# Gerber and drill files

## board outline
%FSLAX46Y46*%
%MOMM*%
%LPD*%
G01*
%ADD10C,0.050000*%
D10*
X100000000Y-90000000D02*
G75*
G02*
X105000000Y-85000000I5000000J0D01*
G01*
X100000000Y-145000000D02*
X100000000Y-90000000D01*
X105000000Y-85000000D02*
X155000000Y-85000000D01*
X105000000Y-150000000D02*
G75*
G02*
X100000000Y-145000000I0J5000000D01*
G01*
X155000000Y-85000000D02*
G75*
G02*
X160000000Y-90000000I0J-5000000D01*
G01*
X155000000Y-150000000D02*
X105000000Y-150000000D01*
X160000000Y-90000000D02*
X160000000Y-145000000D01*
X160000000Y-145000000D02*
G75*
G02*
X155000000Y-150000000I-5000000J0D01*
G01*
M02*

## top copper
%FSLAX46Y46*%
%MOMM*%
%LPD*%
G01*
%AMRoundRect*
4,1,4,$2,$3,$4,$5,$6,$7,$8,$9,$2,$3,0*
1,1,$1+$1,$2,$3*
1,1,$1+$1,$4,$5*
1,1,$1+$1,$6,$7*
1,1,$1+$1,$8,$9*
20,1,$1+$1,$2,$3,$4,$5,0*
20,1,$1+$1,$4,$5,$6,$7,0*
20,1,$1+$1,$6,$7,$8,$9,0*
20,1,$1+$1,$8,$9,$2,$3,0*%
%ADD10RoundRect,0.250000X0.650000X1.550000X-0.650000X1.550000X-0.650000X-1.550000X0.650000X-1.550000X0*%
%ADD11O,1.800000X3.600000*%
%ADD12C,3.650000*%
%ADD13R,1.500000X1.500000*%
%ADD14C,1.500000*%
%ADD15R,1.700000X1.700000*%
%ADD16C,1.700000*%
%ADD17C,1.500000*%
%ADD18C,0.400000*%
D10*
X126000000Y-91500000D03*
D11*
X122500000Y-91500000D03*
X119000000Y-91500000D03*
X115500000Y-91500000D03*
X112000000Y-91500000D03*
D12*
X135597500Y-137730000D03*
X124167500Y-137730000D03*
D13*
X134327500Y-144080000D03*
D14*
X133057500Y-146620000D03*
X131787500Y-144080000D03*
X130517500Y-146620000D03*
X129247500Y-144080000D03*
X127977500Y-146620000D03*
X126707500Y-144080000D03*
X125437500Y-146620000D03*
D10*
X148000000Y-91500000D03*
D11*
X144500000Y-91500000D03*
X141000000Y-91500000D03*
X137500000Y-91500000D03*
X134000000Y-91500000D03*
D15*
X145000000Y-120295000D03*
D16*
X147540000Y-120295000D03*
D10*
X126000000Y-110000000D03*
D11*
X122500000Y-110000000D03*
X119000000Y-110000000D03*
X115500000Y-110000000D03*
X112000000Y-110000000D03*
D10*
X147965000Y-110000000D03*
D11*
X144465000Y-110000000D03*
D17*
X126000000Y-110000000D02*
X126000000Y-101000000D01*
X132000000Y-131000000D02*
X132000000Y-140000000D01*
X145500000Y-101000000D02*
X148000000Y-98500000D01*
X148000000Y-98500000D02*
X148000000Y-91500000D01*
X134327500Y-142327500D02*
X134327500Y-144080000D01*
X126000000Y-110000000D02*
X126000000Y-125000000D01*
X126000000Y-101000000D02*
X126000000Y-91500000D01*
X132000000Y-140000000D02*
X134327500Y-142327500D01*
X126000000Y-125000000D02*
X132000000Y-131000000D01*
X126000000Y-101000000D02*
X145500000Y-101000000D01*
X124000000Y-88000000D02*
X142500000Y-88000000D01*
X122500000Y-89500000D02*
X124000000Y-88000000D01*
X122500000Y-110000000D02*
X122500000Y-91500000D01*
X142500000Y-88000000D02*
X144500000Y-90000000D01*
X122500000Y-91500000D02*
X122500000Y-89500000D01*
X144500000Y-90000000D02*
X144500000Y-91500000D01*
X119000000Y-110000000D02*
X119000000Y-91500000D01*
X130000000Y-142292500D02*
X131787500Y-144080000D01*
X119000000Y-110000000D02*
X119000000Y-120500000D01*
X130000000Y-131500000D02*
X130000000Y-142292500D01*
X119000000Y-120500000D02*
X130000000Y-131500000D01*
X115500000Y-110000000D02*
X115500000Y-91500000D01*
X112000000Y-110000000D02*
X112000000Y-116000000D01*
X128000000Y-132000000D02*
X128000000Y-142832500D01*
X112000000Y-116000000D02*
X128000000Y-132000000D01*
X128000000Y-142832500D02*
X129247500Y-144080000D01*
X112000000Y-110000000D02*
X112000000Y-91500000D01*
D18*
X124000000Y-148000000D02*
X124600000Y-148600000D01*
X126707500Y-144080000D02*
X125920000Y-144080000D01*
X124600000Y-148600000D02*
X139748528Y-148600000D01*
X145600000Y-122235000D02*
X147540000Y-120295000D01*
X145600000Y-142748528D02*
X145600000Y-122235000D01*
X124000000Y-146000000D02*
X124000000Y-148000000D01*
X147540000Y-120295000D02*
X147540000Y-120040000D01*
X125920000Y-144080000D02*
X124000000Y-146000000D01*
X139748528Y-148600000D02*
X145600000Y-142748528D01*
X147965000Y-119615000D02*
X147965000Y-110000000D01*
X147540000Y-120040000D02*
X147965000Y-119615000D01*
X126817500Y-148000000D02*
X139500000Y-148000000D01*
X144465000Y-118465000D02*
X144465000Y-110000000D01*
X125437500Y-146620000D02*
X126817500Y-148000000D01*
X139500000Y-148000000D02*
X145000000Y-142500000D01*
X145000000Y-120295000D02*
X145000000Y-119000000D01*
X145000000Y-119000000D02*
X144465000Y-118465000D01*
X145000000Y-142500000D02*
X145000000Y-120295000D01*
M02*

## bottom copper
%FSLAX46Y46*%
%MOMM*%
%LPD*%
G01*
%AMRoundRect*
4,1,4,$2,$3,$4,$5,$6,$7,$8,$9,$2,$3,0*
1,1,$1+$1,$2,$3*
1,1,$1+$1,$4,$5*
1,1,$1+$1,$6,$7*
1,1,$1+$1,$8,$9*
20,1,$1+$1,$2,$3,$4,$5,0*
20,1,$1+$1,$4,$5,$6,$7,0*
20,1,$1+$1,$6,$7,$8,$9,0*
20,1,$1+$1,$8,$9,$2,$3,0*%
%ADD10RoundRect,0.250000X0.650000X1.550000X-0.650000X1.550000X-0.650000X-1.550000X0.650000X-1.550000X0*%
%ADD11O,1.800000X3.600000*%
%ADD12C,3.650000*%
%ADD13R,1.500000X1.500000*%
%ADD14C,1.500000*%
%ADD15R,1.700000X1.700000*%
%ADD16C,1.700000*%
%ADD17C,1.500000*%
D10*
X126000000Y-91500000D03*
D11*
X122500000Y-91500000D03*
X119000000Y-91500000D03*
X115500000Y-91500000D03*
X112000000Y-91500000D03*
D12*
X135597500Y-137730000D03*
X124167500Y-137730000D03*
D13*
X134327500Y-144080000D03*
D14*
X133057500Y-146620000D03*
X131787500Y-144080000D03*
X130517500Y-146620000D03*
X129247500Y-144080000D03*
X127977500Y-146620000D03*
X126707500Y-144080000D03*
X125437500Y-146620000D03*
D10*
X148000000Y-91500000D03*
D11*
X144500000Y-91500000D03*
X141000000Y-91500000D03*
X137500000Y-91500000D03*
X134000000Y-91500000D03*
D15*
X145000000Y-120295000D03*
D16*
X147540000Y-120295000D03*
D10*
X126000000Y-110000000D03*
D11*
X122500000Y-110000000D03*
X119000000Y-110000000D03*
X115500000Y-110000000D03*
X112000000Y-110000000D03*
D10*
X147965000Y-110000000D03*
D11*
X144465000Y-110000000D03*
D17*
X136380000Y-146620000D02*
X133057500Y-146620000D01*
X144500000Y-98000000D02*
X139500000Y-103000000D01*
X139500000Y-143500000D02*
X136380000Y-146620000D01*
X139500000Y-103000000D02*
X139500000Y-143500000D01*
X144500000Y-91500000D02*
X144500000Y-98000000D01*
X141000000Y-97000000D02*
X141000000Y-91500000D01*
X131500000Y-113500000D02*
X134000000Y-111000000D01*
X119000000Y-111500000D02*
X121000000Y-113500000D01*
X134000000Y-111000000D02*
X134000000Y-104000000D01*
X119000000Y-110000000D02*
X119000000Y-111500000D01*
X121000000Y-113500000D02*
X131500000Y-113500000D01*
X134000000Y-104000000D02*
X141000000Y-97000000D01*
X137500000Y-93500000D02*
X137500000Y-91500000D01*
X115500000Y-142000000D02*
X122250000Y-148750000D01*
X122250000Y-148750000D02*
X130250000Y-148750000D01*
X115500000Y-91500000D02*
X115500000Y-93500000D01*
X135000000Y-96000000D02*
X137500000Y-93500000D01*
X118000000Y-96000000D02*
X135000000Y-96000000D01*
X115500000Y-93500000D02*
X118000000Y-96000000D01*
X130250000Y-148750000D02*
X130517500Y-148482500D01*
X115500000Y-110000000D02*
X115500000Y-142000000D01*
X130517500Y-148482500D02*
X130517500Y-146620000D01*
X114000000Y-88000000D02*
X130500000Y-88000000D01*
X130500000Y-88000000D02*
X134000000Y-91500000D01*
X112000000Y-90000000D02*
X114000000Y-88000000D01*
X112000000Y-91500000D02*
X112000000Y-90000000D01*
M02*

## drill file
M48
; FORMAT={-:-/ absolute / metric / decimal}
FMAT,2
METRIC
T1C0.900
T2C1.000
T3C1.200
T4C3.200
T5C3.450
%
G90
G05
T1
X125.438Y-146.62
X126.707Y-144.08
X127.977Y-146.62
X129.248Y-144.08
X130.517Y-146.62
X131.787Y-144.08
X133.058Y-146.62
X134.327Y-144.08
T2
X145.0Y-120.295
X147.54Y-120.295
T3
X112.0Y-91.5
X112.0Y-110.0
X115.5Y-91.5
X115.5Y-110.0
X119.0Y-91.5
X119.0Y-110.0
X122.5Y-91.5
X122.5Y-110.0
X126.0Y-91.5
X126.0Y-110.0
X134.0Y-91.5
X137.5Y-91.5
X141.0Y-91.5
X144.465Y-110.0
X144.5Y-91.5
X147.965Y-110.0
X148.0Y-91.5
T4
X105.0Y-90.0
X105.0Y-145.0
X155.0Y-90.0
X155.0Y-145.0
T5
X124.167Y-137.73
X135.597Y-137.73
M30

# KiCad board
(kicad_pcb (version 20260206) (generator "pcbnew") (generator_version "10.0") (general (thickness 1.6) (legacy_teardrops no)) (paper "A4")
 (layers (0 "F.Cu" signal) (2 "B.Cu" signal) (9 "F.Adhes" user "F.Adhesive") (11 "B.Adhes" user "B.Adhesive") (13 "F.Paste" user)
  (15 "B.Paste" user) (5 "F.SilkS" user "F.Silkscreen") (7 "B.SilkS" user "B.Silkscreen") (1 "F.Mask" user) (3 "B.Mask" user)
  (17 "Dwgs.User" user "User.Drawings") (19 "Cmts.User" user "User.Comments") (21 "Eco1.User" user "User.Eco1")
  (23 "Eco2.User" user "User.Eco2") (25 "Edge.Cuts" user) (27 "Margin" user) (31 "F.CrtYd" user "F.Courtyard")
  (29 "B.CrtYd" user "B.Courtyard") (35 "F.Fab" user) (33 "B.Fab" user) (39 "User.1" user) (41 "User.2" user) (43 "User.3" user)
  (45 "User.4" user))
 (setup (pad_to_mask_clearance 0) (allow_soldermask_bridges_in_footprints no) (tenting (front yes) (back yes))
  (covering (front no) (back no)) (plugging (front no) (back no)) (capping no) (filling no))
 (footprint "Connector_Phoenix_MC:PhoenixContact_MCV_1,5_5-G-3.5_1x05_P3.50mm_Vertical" (layer "F.Cu") (at 126 91.5 180)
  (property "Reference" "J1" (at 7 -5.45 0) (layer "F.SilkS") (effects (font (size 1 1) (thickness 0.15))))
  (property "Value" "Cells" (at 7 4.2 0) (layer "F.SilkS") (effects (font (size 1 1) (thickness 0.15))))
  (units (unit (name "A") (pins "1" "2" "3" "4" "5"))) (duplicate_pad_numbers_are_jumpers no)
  (pad "1" thru_hole roundrect (at 0 0 180) (size 1.8 3.6) (drill 1.2) (layers "*.Cu" "*.Mask") (remove_unused_layers no)
   (roundrect_rratio 0.138889) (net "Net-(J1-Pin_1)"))
  (pad "2" thru_hole oval (at 3.5 0 180) (size 1.8 3.6) (drill 1.2) (layers "*.Cu" "*.Mask") (remove_unused_layers no)
   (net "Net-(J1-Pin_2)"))
  (pad "3" thru_hole oval (at 7 0 180) (size 1.8 3.6) (drill 1.2) (layers "*.Cu" "*.Mask") (remove_unused_layers no) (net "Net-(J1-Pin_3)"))
  (pad "4" thru_hole oval (at 10.5 0 180) (size 1.8 3.6) (drill 1.2) (layers "*.Cu" "*.Mask") (remove_unused_layers no)
   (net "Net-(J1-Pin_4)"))
  (pad "5" thru_hole oval (at 14 0 180) (size 1.8 3.6) (drill 1.2) (layers "*.Cu" "*.Mask") (remove_unused_layers no) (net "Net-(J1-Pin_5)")))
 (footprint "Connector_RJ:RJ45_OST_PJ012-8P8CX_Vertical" (layer "F.Cu") (at 134.3275 144.08 180)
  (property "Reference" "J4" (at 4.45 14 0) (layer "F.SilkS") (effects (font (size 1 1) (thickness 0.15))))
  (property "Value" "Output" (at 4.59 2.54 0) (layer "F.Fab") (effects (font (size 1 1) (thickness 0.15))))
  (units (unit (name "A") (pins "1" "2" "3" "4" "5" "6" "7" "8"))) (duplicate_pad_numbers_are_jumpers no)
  (pad "" np_thru_hole circle (at -1.27 6.35 180) (size 3.65 3.65) (drill 3.45) (layers "*.Cu" "*.SilkS" "*.Mask"))
  (pad "" np_thru_hole circle (at 10.16 6.35 180) (size 3.65 3.65) (drill 3.45) (layers "*.Cu" "*.SilkS" "*.Mask"))
  (pad "1" thru_hole rect (at 0 0 180) (size 1.5 1.5) (drill 0.9) (layers "*.Cu" "*.Mask") (remove_unused_layers no) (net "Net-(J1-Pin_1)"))
  (pad "2" thru_hole circle (at 1.27 -2.54 180) (size 1.5 1.5) (drill 0.9) (layers "*.Cu" "*.Mask") (remove_unused_layers no)
   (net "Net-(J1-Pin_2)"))
  (pad "3" thru_hole circle (at 2.54 0 180) (size 1.5 1.5) (drill 0.9) (layers "*.Cu" "*.Mask") (remove_unused_layers no)
   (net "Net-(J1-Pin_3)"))
  (pad "4" thru_hole circle (at 3.81 -2.54 180) (size 1.5 1.5) (drill 0.9) (layers "*.Cu" "*.Mask") (remove_unused_layers no)
   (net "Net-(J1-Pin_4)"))
  (pad "5" thru_hole circle (at 5.08 0 180) (size 1.5 1.5) (drill 0.9) (layers "*.Cu" "*.Mask") (remove_unused_layers no)
   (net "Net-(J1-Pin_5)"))
  (pad "6" thru_hole circle (at 6.35 -2.54 180) (size 1.5 1.5) (drill 0.9) (layers "*.Cu" "*.Mask") (remove_unused_layers no)
   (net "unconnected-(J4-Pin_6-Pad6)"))
  (pad "7" thru_hole circle (at 7.62 0 180) (size 1.5 1.5) (drill 0.9) (layers "*.Cu" "*.Mask") (remove_unused_layers no)
   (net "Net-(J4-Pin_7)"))
  (pad "8" thru_hole circle (at 8.89 -2.54 180) (size 1.5 1.5) (drill 0.9) (layers "*.Cu" "*.Mask") (remove_unused_layers no)
   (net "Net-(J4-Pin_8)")))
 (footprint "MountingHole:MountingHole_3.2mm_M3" (layer "F.Cu") (at 105 145)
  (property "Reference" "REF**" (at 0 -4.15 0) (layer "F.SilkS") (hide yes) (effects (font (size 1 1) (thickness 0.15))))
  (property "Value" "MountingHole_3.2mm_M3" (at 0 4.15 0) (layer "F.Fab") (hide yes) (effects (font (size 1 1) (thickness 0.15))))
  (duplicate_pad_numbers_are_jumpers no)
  (pad "" np_thru_hole circle (at 0 0) (size 3.2 3.2) (drill 3.2) (layers "*.Cu" "*.Mask")))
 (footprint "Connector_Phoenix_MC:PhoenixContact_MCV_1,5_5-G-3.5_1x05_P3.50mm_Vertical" (layer "F.Cu") (at 148 91.5 180)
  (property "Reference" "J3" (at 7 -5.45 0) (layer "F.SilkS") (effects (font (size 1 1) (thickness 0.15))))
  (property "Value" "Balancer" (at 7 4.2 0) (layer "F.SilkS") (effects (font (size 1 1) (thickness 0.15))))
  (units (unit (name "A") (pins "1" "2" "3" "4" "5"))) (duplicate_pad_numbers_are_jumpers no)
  (pad "1" thru_hole roundrect (at 0 0 180) (size 1.8 3.6) (drill 1.2) (layers "*.Cu" "*.Mask") (remove_unused_layers no)
   (roundrect_rratio 0.138889) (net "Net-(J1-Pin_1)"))
  (pad "2" thru_hole oval (at 3.5 0 180) (size 1.8 3.6) (drill 1.2) (layers "*.Cu" "*.Mask") (remove_unused_layers no)
   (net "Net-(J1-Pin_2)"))
  (pad "3" thru_hole oval (at 7 0 180) (size 1.8 3.6) (drill 1.2) (layers "*.Cu" "*.Mask") (remove_unused_layers no) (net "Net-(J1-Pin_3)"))
  (pad "4" thru_hole oval (at 10.5 0 180) (size 1.8 3.6) (drill 1.2) (layers "*.Cu" "*.Mask") (remove_unused_layers no)
   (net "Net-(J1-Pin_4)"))
  (pad "5" thru_hole oval (at 14 0 180) (size 1.8 3.6) (drill 1.2) (layers "*.Cu" "*.Mask") (remove_unused_layers no) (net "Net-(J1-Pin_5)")))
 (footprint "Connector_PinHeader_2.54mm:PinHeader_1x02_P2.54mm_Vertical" (layer "F.Cu") (at 145 120.295 90)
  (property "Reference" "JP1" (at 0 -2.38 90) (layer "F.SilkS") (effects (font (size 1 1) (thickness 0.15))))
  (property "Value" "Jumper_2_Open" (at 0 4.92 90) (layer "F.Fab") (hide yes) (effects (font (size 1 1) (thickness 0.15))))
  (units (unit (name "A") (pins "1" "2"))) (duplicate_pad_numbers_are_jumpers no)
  (pad "1" thru_hole rect (at 0 0 90) (size 1.7 1.7) (drill 1) (layers "*.Cu" "*.Mask") (remove_unused_layers no) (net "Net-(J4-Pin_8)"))
  (pad "2" thru_hole circle (at 0 2.54 90) (size 1.7 1.7) (drill 1) (layers "*.Cu" "*.Mask") (remove_unused_layers no)
   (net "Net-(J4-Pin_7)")))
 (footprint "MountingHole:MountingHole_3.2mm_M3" (layer "F.Cu") (at 105 90)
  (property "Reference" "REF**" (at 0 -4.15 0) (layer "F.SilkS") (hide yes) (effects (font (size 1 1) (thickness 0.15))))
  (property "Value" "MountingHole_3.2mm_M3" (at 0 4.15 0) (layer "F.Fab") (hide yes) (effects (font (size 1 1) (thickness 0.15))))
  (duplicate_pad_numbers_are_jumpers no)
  (pad "" np_thru_hole circle (at 0 0) (size 3.2 3.2) (drill 3.2) (layers "*.Cu" "*.Mask")))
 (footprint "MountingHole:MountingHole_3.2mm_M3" (layer "F.Cu") (at 155 90)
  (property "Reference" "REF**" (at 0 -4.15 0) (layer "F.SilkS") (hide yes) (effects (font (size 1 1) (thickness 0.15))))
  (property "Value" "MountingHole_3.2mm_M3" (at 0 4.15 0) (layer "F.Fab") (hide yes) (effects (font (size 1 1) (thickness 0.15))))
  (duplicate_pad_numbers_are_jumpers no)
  (pad "" np_thru_hole circle (at 0 0) (size 3.2 3.2) (drill 3.2) (layers "*.Cu" "*.Mask")))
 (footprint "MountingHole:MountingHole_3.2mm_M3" (layer "F.Cu") (at 155 145)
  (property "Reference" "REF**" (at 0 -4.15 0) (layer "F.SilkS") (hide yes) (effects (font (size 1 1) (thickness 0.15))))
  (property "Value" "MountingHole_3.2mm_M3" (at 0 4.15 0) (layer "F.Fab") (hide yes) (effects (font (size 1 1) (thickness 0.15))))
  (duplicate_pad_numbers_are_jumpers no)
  (pad "" np_thru_hole circle (at 0 0) (size 3.2 3.2) (drill 3.2) (layers "*.Cu" "*.Mask")))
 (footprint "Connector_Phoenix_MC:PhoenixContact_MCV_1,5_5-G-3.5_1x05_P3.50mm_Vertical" (layer "F.Cu") (at 126 110 180)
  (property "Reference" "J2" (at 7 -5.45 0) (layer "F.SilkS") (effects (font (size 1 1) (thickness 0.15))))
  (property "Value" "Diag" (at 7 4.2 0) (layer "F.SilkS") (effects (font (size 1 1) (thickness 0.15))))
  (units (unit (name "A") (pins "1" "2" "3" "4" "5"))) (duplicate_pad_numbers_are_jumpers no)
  (pad "1" thru_hole roundrect (at 0 0 180) (size 1.8 3.6) (drill 1.2) (layers "*.Cu" "*.Mask") (remove_unused_layers no)
   (roundrect_rratio 0.138889) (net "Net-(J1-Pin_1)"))
  (pad "2" thru_hole oval (at 3.5 0 180) (size 1.8 3.6) (drill 1.2) (layers "*.Cu" "*.Mask") (remove_unused_layers no)
   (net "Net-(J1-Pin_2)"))
  (pad "3" thru_hole oval (at 7 0 180) (size 1.8 3.6) (drill 1.2) (layers "*.Cu" "*.Mask") (remove_unused_layers no) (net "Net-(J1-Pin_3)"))
  (pad "4" thru_hole oval (at 10.5 0 180) (size 1.8 3.6) (drill 1.2) (layers "*.Cu" "*.Mask") (remove_unused_layers no)
   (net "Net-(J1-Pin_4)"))
  (pad "5" thru_hole oval (at 14 0 180) (size 1.8 3.6) (drill 1.2) (layers "*.Cu" "*.Mask") (remove_unused_layers no) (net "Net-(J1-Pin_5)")))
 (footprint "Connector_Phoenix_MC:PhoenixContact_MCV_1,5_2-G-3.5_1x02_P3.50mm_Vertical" (layer "F.Cu") (at 147.965 110 180)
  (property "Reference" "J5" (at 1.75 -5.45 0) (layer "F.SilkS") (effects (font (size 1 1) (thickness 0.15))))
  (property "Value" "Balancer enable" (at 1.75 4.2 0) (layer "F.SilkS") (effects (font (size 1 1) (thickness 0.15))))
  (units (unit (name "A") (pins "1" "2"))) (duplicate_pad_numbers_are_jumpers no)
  (pad "1" thru_hole roundrect (at 0 0 180) (size 1.8 3.6) (drill 1.2) (layers "*.Cu" "*.Mask") (remove_unused_layers no)
   (roundrect_rratio 0.138889) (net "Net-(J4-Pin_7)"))
  (pad "2" thru_hole oval (at 3.5 0 180) (size 1.8 3.6) (drill 1.2) (layers "*.Cu" "*.Mask") (remove_unused_layers no)
   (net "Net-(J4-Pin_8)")))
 (gr_arc (start 100 90) (mid 101.464466 86.464466) (end 105 85) (stroke (width 0.05) (type default)) (layer "Edge.Cuts"))
 (gr_line (start 100 145) (end 100 90) (stroke (width 0.05) (type default)) (layer "Edge.Cuts"))
 (gr_line (start 105 85) (end 155 85) (stroke (width 0.05) (type default)) (layer "Edge.Cuts"))
 (gr_arc (start 105 150) (mid 101.464466 148.535534) (end 100 145) (stroke (width 0.05) (type default)) (layer "Edge.Cuts"))
 (gr_arc (start 155 85) (mid 158.535534 86.464466) (end 160 90) (stroke (width 0.05) (type default)) (layer "Edge.Cuts"))
 (gr_line (start 155 150) (end 105 150) (stroke (width 0.05) (type default)) (layer "Edge.Cuts"))
 (gr_line (start 160 90) (end 160 145) (stroke (width 0.05) (type default)) (layer "Edge.Cuts"))
 (gr_arc (start 160 145) (mid 158.535534 148.535534) (end 155 150) (stroke (width 0.05) (type default)) (layer "Edge.Cuts"))
 (segment (start 126 110) (end 126 101) (width 1.5) (layer "F.Cu") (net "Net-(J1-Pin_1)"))
 (segment (start 132 131) (end 132 140) (width 1.5) (layer "F.Cu") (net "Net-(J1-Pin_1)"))
 (segment (start 145.5 101) (end 148 98.5) (width 1.5) (layer "F.Cu") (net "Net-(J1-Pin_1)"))
 (segment (start 148 98.5) (end 148 91.5) (width 1.5) (layer "F.Cu") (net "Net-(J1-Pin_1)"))
 (segment (start 134.3275 142.3275) (end 134.3275 144.08) (width 1.5) (layer "F.Cu") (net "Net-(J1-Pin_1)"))
 (segment (start 126 110) (end 126 125) (width 1.5) (layer "F.Cu") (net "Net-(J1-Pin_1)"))
 (segment (start 126 101) (end 126 91.5) (width 1.5) (layer "F.Cu") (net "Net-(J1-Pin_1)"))
 (segment (start 132 140) (end 134.3275 142.3275) (width 1.5) (layer "F.Cu") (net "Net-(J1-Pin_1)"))
 (segment (start 126 125) (end 132 131) (width 1.5) (layer "F.Cu") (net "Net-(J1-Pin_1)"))
 (segment (start 126 101) (end 145.5 101) (width 1.5) (layer "F.Cu") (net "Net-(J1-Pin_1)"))
 (segment (start 124 88) (end 142.5 88) (width 1.5) (layer "F.Cu") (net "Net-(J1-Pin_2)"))
 (segment (start 122.5 89.5) (end 124 88) (width 1.5) (layer "F.Cu") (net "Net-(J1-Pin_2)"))
 (segment (start 122.5 110) (end 122.5 91.5) (width 1.5) (layer "F.Cu") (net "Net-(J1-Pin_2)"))
 (segment (start 142.5 88) (end 144.5 90) (width 1.5) (layer "F.Cu") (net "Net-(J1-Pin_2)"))
 (segment (start 122.5 91.5) (end 122.5 89.5) (width 1.5) (layer "F.Cu") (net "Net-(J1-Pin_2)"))
 (segment (start 144.5 90) (end 144.5 91.5) (width 1.5) (layer "F.Cu") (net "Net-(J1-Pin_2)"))
 (segment (start 136.38 146.62) (end 133.0575 146.62) (width 1.5) (layer "B.Cu") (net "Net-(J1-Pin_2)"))
 (segment (start 144.5 98) (end 139.5 103) (width 1.5) (layer "B.Cu") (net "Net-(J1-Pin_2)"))
 (segment (start 139.5 143.5) (end 136.38 146.62) (width 1.5) (layer "B.Cu") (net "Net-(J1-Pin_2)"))
 (segment (start 139.5 103) (end 139.5 143.5) (width 1.5) (layer "B.Cu") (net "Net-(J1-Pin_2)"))
 (segment (start 144.5 91.5) (end 144.5 98) (width 1.5) (layer "B.Cu") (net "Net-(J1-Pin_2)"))
 (segment (start 119 110) (end 119 91.5) (width 1.5) (layer "F.Cu") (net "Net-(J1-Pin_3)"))
 (segment (start 130 142.2925) (end 131.7875 144.08) (width 1.5) (layer "F.Cu") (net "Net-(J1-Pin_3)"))
 (segment (start 119 110) (end 119 120.5) (width 1.5) (layer "F.Cu") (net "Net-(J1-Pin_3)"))
 (segment (start 130 131.5) (end 130 142.2925) (width 1.5) (layer "F.Cu") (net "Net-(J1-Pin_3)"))
 (segment (start 119 120.5) (end 130 131.5) (width 1.5) (layer "F.Cu") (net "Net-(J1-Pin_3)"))
 (segment (start 141 97) (end 141 91.5) (width 1.5) (layer "B.Cu") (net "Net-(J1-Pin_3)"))
 (segment (start 131.5 113.5) (end 134 111) (width 1.5) (layer "B.Cu") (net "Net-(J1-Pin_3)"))
 (segment (start 119 111.5) (end 121 113.5) (width 1.5) (layer "B.Cu") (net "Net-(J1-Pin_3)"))
 (segment (start 134 111) (end 134 104) (width 1.5) (layer "B.Cu") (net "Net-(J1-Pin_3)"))
 (segment (start 119 110) (end 119 111.5) (width 1.5) (layer "B.Cu") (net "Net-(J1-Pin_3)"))
 (segment (start 121 113.5) (end 131.5 113.5) (width 1.5) (layer "B.Cu") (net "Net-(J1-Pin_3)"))
 (segment (start 134 104) (end 141 97) (width 1.5) (layer "B.Cu") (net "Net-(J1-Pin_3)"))
 (segment (start 115.5 110) (end 115.5 91.5) (width 1.5) (layer "F.Cu") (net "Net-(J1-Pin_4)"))
 (segment (start 137.5 93.5) (end 137.5 91.5) (width 1.5) (layer "B.Cu") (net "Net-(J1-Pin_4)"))
 (segment (start 115.5 142) (end 122.25 148.75) (width 1.5) (layer "B.Cu") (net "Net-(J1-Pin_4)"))
 (segment (start 122.25 148.75) (end 130.25 148.75) (width 1.5) (layer "B.Cu") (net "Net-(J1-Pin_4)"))
 (segment (start 115.5 91.5) (end 115.5 93.5) (width 1.5) (layer "B.Cu") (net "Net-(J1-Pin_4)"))
 (segment (start 135 96) (end 137.5 93.5) (width 1.5) (layer "B.Cu") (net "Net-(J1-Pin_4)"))
 (segment (start 118 96) (end 135 96) (width 1.5) (layer "B.Cu") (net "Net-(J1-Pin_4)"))
 (segment (start 115.5 93.5) (end 118 96) (width 1.5) (layer "B.Cu") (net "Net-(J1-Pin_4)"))
 (segment (start 130.25 148.75) (end 130.5175 148.4825) (width 1.5) (layer "B.Cu") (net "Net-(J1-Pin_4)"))
 (segment (start 115.5 110) (end 115.5 142) (width 1.5) (layer "B.Cu") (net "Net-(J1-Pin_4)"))
 (segment (start 130.5175 148.4825) (end 130.5175 146.62) (width 1.5) (layer "B.Cu") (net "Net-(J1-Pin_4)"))
 (segment (start 112 110) (end 112 116) (width 1.5) (layer "F.Cu") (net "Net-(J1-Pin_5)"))
 (segment (start 128 132) (end 128 142.8325) (width 1.5) (layer "F.Cu") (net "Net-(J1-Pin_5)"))
 (segment (start 112 116) (end 128 132) (width 1.5) (layer "F.Cu") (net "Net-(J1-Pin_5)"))
 (segment (start 128 142.8325) (end 129.2475 144.08) (width 1.5) (layer "F.Cu") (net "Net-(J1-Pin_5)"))
 (segment (start 112 110) (end 112 91.5) (width 1.5) (layer "F.Cu") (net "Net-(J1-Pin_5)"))
 (segment (start 114 88) (end 130.5 88) (width 1.5) (layer "B.Cu") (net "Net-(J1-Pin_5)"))
 (segment (start 130.5 88) (end 134 91.5) (width 1.5) (layer "B.Cu") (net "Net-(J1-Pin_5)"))
 (segment (start 112 90) (end 114 88) (width 1.5) (layer "B.Cu") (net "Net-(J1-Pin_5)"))
 (segment (start 112 91.5) (end 112 90) (width 1.5) (layer "B.Cu") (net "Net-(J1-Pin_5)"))
 (segment (start 124 148) (end 124.6 148.6) (width 0.4) (layer "F.Cu") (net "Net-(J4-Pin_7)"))
 (segment (start 126.7075 144.08) (end 125.92 144.08) (width 0.4) (layer "F.Cu") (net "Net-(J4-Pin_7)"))
 (segment (start 124.6 148.6) (end 139.748528 148.6) (width 0.4) (layer "F.Cu") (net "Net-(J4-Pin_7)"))
 (segment (start 145.6 122.235) (end 147.54 120.295) (width 0.4) (layer "F.Cu") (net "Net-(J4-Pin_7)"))
 (segment (start 145.6 142.748528) (end 145.6 122.235) (width 0.4) (layer "F.Cu") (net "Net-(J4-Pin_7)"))
 (segment (start 124 146) (end 124 148) (width 0.4) (layer "F.Cu") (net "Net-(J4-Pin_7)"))
 (segment (start 147.54 120.295) (end 147.54 120.04) (width 0.4) (layer "F.Cu") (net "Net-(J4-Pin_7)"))
 (segment (start 125.92 144.08) (end 124 146) (width 0.4) (layer "F.Cu") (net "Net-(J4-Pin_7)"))
 (segment (start 139.748528 148.6) (end 145.6 142.748528) (width 0.4) (layer "F.Cu") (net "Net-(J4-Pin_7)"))
 (segment (start 147.965 119.615) (end 147.965 110) (width 0.4) (layer "F.Cu") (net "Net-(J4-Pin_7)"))
 (segment (start 147.54 120.04) (end 147.965 119.615) (width 0.4) (layer "F.Cu") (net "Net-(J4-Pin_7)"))
 (segment (start 126.8175 148) (end 139.5 148) (width 0.4) (layer "F.Cu") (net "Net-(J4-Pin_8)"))
 (segment (start 144.465 118.465) (end 144.465 110) (width 0.4) (layer "F.Cu") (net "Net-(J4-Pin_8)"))
 (segment (start 125.4375 146.62) (end 126.8175 148) (width 0.4) (layer "F.Cu") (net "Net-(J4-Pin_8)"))
 (segment (start 139.5 148) (end 145 142.5) (width 0.4) (layer "F.Cu") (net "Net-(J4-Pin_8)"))
 (segment (start 145 120.295) (end 145 119) (width 0.4) (layer "F.Cu") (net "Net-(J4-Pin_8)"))
 (segment (start 145 119) (end 144.465 118.465) (width 0.4) (layer "F.Cu") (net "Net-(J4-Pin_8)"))
 (segment (start 145 142.5) (end 145 120.295) (width 0.4) (layer "F.Cu") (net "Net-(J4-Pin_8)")))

